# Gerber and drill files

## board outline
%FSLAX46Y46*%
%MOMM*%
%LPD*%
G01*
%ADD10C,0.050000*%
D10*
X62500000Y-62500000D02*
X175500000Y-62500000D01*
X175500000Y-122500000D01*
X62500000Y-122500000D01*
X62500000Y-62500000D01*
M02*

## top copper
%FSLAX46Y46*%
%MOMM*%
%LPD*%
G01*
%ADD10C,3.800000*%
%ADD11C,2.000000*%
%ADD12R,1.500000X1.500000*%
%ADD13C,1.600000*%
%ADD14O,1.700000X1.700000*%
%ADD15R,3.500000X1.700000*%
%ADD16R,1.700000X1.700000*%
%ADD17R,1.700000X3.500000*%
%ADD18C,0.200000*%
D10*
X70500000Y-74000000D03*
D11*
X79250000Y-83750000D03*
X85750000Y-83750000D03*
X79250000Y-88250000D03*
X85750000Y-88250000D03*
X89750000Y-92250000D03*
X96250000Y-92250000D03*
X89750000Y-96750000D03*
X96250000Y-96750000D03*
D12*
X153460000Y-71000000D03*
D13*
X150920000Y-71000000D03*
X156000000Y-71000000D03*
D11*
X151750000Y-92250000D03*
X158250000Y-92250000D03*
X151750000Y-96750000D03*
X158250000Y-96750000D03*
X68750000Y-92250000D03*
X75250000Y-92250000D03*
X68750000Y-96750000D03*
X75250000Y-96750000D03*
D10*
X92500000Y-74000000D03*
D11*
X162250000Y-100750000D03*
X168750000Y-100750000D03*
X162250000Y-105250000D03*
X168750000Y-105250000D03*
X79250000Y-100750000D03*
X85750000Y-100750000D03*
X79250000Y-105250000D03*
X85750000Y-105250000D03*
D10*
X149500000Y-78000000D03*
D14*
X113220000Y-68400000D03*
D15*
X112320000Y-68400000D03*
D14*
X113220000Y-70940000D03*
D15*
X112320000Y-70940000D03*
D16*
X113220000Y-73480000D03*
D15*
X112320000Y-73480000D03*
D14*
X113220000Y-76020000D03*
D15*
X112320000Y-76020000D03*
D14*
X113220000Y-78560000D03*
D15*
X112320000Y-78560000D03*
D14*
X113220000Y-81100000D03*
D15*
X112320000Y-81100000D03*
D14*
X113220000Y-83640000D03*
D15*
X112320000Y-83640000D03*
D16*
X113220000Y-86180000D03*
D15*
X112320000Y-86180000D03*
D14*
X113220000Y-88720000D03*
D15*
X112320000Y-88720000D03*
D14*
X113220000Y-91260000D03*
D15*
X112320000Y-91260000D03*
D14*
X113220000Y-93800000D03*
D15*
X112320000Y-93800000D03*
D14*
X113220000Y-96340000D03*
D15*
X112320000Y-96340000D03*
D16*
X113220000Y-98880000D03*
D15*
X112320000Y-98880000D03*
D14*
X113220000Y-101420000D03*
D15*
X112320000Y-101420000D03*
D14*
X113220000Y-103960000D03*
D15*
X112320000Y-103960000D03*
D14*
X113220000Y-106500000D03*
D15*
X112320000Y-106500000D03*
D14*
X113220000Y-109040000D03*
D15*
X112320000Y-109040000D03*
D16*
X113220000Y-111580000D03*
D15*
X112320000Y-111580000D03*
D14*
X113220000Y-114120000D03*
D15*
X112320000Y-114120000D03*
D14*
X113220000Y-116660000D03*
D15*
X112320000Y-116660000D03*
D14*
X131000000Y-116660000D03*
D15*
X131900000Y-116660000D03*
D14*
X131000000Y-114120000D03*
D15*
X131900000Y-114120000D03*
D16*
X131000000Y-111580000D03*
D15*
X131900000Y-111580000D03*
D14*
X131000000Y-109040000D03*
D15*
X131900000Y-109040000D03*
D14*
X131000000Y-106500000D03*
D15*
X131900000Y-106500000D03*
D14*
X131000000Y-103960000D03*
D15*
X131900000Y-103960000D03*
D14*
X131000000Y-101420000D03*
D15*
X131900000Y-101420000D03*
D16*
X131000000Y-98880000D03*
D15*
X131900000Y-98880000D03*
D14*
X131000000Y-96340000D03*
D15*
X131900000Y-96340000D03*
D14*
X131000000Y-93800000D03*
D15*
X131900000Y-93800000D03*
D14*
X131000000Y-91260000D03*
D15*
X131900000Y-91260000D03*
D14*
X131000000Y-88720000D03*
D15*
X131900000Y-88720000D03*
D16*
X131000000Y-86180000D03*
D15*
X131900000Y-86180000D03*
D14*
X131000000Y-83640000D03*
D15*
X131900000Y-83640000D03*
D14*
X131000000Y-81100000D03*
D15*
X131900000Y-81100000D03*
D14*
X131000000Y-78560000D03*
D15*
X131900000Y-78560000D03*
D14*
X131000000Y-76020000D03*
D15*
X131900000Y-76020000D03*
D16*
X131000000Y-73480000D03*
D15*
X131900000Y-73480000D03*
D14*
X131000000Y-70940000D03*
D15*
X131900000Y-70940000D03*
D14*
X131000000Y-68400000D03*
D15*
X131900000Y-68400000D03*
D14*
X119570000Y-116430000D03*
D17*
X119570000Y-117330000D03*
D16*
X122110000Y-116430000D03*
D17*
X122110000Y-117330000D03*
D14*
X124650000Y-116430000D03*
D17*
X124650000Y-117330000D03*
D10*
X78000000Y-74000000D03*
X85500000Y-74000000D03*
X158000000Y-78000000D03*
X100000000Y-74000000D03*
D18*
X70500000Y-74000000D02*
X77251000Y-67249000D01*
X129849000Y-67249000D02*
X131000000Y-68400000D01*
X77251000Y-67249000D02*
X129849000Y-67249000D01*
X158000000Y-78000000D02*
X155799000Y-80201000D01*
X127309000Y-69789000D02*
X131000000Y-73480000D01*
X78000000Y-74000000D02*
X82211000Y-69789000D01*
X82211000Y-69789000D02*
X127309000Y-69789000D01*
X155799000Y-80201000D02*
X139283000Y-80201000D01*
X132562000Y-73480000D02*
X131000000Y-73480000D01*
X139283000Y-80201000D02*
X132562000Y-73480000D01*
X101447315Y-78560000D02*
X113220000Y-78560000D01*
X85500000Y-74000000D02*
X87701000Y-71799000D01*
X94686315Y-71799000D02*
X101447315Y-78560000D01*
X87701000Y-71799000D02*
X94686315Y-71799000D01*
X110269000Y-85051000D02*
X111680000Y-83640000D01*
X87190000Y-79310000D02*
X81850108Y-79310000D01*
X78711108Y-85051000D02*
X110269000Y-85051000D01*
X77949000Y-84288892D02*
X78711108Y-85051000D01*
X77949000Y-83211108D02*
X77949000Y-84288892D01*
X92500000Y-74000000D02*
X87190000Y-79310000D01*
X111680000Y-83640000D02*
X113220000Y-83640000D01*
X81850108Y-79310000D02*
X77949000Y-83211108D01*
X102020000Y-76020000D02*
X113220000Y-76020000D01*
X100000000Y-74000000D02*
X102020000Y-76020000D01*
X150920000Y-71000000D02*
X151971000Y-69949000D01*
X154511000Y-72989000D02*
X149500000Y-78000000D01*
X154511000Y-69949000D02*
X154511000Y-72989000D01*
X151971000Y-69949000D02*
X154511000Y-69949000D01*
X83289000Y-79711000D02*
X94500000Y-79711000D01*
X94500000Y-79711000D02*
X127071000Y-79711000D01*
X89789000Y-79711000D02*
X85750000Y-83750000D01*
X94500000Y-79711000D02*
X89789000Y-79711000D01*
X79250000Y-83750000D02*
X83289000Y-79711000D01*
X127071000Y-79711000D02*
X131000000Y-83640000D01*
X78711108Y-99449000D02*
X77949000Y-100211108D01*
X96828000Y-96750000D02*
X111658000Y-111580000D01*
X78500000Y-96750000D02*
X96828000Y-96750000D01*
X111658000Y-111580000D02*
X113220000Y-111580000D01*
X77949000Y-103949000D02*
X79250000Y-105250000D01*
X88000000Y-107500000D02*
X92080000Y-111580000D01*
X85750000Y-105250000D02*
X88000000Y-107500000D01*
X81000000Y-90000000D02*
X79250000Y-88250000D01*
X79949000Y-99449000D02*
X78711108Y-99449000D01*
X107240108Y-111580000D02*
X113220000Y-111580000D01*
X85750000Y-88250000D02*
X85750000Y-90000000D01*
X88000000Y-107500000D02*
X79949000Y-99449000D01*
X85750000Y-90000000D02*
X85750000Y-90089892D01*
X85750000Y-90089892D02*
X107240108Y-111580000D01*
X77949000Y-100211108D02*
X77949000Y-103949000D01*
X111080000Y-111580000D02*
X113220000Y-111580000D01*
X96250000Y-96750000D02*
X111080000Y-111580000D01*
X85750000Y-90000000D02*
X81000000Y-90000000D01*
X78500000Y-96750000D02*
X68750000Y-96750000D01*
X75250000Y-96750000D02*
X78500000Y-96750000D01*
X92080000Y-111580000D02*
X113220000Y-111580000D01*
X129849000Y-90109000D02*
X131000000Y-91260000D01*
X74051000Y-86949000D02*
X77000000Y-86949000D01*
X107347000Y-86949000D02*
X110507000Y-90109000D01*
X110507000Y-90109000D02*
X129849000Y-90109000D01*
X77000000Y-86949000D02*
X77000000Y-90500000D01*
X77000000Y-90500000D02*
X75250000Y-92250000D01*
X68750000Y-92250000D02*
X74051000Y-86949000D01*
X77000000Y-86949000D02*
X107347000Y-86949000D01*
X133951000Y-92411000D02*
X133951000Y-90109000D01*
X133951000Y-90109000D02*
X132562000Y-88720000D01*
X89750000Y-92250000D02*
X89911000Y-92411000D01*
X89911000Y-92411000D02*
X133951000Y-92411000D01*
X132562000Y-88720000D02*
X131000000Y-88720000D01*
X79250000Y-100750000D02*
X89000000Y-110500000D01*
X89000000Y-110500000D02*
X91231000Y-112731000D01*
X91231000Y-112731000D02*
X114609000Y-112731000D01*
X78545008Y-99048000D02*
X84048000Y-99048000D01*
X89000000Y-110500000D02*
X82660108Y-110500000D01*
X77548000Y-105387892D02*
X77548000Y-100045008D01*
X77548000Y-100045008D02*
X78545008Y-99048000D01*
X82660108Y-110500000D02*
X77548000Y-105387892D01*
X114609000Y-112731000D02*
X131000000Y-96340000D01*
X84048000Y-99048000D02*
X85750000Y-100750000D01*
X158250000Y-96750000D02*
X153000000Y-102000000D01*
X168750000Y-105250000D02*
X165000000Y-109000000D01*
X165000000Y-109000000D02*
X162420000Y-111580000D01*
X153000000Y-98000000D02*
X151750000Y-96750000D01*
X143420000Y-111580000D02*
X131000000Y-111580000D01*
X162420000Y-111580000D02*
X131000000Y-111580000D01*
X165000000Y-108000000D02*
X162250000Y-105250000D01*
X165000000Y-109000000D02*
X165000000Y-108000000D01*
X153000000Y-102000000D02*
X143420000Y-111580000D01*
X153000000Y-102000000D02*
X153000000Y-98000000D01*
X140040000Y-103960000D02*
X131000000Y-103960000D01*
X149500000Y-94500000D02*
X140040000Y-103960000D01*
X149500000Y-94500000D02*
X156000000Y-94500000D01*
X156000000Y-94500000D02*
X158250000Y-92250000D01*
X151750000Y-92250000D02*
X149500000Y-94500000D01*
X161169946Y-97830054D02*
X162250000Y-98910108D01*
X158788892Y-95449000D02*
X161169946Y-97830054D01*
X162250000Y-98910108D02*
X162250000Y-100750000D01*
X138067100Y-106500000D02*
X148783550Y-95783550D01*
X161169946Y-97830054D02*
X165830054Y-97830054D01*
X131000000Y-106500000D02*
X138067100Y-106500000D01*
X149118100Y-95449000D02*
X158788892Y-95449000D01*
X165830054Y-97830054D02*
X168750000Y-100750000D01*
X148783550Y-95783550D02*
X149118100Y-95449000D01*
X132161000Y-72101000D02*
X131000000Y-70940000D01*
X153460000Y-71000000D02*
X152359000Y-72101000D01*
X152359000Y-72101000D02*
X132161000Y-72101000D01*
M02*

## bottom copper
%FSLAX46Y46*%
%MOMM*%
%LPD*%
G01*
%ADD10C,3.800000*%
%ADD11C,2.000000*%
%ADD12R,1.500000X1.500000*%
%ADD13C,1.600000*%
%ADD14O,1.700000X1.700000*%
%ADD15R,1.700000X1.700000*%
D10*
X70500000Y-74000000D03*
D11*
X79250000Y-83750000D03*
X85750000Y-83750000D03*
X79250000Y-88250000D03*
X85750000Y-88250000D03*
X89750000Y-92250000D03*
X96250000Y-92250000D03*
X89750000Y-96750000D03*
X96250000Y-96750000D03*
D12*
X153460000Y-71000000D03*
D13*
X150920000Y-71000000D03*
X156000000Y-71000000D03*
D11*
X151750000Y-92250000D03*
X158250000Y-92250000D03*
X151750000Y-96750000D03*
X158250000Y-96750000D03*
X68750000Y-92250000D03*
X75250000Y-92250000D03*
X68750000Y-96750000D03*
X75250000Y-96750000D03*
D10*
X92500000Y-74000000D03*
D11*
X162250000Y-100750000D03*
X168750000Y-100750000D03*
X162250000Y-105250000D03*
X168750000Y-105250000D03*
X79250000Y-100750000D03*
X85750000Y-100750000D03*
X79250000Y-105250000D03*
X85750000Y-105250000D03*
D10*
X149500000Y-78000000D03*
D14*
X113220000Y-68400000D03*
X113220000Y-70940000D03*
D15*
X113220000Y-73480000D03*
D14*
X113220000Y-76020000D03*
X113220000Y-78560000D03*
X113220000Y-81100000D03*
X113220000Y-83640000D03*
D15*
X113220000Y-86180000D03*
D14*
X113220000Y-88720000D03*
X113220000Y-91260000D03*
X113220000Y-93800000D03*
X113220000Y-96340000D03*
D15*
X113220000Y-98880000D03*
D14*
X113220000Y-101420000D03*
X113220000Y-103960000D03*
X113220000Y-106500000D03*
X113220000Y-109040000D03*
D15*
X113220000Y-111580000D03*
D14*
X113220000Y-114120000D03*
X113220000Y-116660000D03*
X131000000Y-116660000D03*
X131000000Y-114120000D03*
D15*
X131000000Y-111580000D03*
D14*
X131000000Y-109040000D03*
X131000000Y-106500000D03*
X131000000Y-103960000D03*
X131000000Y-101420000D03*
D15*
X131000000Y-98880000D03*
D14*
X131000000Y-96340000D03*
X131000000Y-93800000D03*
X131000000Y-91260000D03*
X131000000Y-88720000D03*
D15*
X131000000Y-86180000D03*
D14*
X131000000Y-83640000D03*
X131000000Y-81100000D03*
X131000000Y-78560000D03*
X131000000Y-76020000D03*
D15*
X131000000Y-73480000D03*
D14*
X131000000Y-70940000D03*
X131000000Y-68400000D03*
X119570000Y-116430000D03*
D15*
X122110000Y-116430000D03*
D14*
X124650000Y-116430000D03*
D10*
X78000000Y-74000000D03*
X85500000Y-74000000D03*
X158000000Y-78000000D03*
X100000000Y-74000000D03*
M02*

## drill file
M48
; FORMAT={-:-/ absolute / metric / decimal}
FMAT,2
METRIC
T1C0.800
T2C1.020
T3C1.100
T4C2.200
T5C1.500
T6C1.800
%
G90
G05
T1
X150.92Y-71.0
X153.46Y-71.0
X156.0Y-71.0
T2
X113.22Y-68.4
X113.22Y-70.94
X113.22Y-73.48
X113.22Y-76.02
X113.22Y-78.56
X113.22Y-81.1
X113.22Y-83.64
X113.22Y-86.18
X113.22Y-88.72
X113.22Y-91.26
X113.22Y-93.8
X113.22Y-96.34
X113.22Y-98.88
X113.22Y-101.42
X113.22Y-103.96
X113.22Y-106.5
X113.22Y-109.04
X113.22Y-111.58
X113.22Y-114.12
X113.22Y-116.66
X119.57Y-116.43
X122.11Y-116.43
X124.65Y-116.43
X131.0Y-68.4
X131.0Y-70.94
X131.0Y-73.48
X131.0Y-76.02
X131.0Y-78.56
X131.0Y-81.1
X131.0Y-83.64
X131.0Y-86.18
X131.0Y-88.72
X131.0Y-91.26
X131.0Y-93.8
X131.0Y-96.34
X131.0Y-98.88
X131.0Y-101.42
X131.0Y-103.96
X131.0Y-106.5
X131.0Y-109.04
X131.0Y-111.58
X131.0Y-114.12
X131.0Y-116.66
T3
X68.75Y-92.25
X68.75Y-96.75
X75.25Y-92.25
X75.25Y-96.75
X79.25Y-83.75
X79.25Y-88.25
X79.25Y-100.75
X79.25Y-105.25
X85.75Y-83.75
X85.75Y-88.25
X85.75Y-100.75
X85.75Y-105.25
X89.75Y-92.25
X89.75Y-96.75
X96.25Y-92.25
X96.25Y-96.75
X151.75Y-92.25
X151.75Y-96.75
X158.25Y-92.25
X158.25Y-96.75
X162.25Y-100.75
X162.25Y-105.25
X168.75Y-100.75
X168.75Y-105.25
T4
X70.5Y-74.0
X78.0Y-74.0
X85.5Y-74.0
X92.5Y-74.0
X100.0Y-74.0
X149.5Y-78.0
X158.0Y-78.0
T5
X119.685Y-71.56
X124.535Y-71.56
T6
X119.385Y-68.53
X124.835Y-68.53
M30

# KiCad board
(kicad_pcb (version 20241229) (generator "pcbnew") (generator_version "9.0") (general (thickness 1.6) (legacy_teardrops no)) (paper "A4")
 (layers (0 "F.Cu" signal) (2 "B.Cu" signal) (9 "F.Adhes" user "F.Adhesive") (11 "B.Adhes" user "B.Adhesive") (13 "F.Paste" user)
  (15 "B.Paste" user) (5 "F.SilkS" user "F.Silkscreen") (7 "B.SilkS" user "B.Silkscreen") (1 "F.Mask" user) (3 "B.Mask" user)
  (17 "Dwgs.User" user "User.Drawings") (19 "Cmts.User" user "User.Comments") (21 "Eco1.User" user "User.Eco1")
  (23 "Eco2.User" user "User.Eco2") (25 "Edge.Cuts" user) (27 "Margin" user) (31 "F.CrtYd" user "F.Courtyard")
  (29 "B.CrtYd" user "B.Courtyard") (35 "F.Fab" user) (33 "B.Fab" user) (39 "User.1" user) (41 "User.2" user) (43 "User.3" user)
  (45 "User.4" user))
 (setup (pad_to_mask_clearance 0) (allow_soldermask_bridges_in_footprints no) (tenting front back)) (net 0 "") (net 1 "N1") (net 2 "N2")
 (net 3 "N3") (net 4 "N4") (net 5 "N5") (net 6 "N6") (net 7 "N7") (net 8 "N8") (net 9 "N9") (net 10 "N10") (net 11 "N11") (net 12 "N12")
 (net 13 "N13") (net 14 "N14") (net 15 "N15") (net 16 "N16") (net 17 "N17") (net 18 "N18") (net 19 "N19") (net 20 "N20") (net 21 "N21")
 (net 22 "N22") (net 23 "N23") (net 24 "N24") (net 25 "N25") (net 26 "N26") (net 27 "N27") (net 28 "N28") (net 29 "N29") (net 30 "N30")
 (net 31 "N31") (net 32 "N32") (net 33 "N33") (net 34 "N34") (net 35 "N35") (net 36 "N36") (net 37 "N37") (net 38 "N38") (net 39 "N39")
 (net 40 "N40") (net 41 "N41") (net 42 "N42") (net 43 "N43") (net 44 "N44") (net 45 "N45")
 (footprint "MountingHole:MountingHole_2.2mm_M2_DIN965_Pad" (layer "F.Cu") (at 70.5 74)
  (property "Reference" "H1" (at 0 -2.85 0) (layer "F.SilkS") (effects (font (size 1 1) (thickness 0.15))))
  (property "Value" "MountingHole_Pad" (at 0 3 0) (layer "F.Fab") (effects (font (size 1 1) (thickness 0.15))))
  (pad "1" thru_hole circle (at 0 0) (size 3.8 3.8) (drill 2.2) (layers "*.Cu" "*.Mask") (remove_unused_layers no) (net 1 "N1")
   (zone_connect 2)))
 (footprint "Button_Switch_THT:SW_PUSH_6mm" (layer "F.Cu") (at 79.25 83.75)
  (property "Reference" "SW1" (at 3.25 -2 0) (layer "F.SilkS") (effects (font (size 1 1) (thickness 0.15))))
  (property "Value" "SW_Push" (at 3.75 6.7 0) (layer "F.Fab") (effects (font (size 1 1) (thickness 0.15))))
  (pad "1" thru_hole circle (at 0 0 90) (size 2 2) (drill 1.1) (layers "*.Cu" "*.Mask") (remove_unused_layers no) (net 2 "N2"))
  (pad "1" thru_hole circle (at 6.5 0 90) (size 2 2) (drill 1.1) (layers "*.Cu" "*.Mask") (remove_unused_layers no) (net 2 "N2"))
  (pad "2" thru_hole circle (at 0 4.5 90) (size 2 2) (drill 1.1) (layers "*.Cu" "*.Mask") (remove_unused_layers no) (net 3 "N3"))
  (pad "2" thru_hole circle (at 6.5 4.5 90) (size 2 2) (drill 1.1) (layers "*.Cu" "*.Mask") (remove_unused_layers no) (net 3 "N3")))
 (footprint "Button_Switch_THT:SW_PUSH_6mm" (layer "F.Cu") (at 89.75 92.25)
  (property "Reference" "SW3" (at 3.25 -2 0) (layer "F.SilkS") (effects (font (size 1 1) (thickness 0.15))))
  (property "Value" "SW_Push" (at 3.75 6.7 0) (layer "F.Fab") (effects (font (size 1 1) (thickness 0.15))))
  (pad "1" thru_hole circle (at 0 0 90) (size 2 2) (drill 1.1) (layers "*.Cu" "*.Mask") (remove_unused_layers no) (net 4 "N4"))
  (pad "1" thru_hole circle (at 6.5 0 90) (size 2 2) (drill 1.1) (layers "*.Cu" "*.Mask") (remove_unused_layers no) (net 4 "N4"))
  (pad "2" thru_hole circle (at 0 4.5 90) (size 2 2) (drill 1.1) (layers "*.Cu" "*.Mask") (remove_unused_layers no) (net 3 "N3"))
  (pad "2" thru_hole circle (at 6.5 4.5 90) (size 2 2) (drill 1.1) (layers "*.Cu" "*.Mask") (remove_unused_layers no) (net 3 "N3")))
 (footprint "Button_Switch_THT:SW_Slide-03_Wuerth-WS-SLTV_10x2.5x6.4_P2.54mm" (layer "F.Cu") (at 153.46 71)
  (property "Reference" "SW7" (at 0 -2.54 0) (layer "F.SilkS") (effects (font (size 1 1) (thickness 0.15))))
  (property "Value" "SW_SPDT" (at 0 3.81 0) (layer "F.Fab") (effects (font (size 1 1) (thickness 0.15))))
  (pad "1" thru_hole rect (at 0 0) (size 1.5 1.5) (drill 0.8) (layers "*.Cu" "*.Mask") (remove_unused_layers no) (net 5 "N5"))
  (pad "2" thru_hole circle (at -2.54 0) (size 1.6 1.6) (drill 0.8) (layers "*.Cu" "*.Mask") (remove_unused_layers no) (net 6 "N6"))
  (pad "3" thru_hole circle (at 2.54 0) (size 1.6 1.6) (drill 0.8) (layers "*.Cu" "*.Mask") (remove_unused_layers no) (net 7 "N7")))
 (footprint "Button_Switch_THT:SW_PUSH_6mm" (layer "F.Cu") (at 151.75 92.25)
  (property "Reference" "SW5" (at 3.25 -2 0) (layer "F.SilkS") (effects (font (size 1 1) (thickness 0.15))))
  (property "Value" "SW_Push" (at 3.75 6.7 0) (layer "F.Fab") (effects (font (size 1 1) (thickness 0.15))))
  (pad "1" thru_hole circle (at 0 0 90) (size 2 2) (drill 1.1) (layers "*.Cu" "*.Mask") (remove_unused_layers no) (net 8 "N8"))
  (pad "1" thru_hole circle (at 6.5 0 90) (size 2 2) (drill 1.1) (layers "*.Cu" "*.Mask") (remove_unused_layers no) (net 8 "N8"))
  (pad "2" thru_hole circle (at 0 4.5 90) (size 2 2) (drill 1.1) (layers "*.Cu" "*.Mask") (remove_unused_layers no) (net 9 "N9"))
  (pad "2" thru_hole circle (at 6.5 4.5 90) (size 2 2) (drill 1.1) (layers "*.Cu" "*.Mask") (remove_unused_layers no) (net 9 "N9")))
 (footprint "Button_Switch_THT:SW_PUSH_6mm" (layer "F.Cu") (at 68.75 92.25)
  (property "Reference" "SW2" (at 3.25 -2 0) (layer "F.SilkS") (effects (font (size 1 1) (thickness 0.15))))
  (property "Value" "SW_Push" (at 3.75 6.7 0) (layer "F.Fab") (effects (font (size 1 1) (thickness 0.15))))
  (pad "1" thru_hole circle (at 0 0 90) (size 2 2) (drill 1.1) (layers "*.Cu" "*.Mask") (remove_unused_layers no) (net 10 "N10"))
  (pad "1" thru_hole circle (at 6.5 0 90) (size 2 2) (drill 1.1) (layers "*.Cu" "*.Mask") (remove_unused_layers no) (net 10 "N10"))
  (pad "2" thru_hole circle (at 0 4.5 90) (size 2 2) (drill 1.1) (layers "*.Cu" "*.Mask") (remove_unused_layers no) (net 3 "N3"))
  (pad "2" thru_hole circle (at 6.5 4.5 90) (size 2 2) (drill 1.1) (layers "*.Cu" "*.Mask") (remove_unused_layers no) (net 3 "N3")))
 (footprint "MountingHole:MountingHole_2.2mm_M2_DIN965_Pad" (layer "F.Cu") (at 92.5 74)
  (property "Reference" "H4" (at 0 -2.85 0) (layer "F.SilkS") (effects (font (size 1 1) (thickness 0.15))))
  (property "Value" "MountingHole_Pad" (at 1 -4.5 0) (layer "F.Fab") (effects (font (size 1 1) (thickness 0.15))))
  (pad "1" thru_hole circle (at 0 0) (size 3.8 3.8) (drill 2.2) (layers "*.Cu" "*.Mask") (remove_unused_layers no) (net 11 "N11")
   (zone_connect 2)))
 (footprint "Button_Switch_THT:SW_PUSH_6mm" (layer "F.Cu") (at 162.25 100.75)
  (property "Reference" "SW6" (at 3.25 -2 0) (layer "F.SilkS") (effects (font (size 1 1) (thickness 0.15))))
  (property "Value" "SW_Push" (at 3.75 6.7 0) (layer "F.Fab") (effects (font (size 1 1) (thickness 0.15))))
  (pad "1" thru_hole circle (at 0 0 90) (size 2 2) (drill 1.1) (layers "*.Cu" "*.Mask") (remove_unused_layers no) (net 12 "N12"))
  (pad "1" thru_hole circle (at 6.5 0 90) (size 2 2) (drill 1.1) (layers "*.Cu" "*.Mask") (remove_unused_layers no) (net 12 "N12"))
  (pad "2" thru_hole circle (at 0 4.5 90) (size 2 2) (drill 1.1) (layers "*.Cu" "*.Mask") (remove_unused_layers no) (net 9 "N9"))
  (pad "2" thru_hole circle (at 6.5 4.5 90) (size 2 2) (drill 1.1) (layers "*.Cu" "*.Mask") (remove_unused_layers no) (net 9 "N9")))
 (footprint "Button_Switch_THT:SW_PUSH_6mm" (layer "F.Cu") (at 79.25 100.75)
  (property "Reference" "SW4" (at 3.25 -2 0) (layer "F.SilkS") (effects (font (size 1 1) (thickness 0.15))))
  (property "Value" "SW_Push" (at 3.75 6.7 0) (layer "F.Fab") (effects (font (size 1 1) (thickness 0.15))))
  (pad "1" thru_hole circle (at 0 0 90) (size 2 2) (drill 1.1) (layers "*.Cu" "*.Mask") (remove_unused_layers no) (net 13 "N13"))
  (pad "1" thru_hole circle (at 6.5 0 90) (size 2 2) (drill 1.1) (layers "*.Cu" "*.Mask") (remove_unused_layers no) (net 13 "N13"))
  (pad "2" thru_hole circle (at 0 4.5 90) (size 2 2) (drill 1.1) (layers "*.Cu" "*.Mask") (remove_unused_layers no) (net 3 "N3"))
  (pad "2" thru_hole circle (at 6.5 4.5 90) (size 2 2) (drill 1.1) (layers "*.Cu" "*.Mask") (remove_unused_layers no) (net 3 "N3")))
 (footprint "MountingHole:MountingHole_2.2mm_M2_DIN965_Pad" (layer "F.Cu") (at 149.5 78)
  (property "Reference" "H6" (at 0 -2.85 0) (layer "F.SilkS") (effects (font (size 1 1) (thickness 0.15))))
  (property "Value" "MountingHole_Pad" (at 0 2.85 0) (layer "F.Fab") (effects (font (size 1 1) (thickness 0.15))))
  (pad "1" thru_hole circle (at 0 0) (size 3.8 3.8) (drill 2.2) (layers "*.Cu" "*.Mask") (remove_unused_layers no) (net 6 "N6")
   (zone_connect 2)))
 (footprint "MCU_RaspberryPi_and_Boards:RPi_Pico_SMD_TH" (layer "F.Cu") (at 122.11 92.53)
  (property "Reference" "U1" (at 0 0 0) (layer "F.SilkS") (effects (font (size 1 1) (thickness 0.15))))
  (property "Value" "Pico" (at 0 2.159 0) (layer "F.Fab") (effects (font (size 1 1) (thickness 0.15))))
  (pad "" np_thru_hole oval (at -2.725 -24) (size 1.8 1.8) (drill 1.8) (layers "*.Cu" "*.Mask"))
  (pad "" np_thru_hole oval (at -2.425 -20.97) (size 1.5 1.5) (drill 1.5) (layers "*.Cu" "*.Mask"))
  (pad "" np_thru_hole oval (at 2.425 -20.97) (size 1.5 1.5) (drill 1.5) (layers "*.Cu" "*.Mask"))
  (pad "" np_thru_hole oval (at 2.725 -24) (size 1.8 1.8) (drill 1.8) (layers "*.Cu" "*.Mask"))
  (pad "1" thru_hole oval (at -8.89 -24.13) (size 1.7 1.7) (drill 1.02) (layers "*.Cu" "*.Mask") (remove_unused_layers no) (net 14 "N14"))
  (pad "1" smd rect (at -8.89 -24.13) (size 3.5 1.7) (drill (offset -0.9 0)) (layers "F.Cu" "F.Mask") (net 14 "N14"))
  (pad "2" thru_hole oval (at -8.89 -21.59) (size 1.7 1.7) (drill 1.02) (layers "*.Cu" "*.Mask") (remove_unused_layers no) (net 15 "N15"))
  (pad "2" smd rect (at -8.89 -21.59) (size 3.5 1.7) (drill (offset -0.9 0)) (layers "F.Cu" "F.Mask") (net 15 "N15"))
  (pad "3" thru_hole rect (at -8.89 -19.05) (size 1.7 1.7) (drill 1.02) (layers "*.Cu" "*.Mask") (remove_unused_layers no) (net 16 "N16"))
  (pad "3" smd rect (at -8.89 -19.05) (size 3.5 1.7) (drill (offset -0.9 0)) (layers "F.Cu" "F.Mask") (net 16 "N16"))
  (pad "4" thru_hole oval (at -8.89 -16.51) (size 1.7 1.7) (drill 1.02) (layers "*.Cu" "*.Mask") (remove_unused_layers no) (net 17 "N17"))
  (pad "4" smd rect (at -8.89 -16.51) (size 3.5 1.7) (drill (offset -0.9 0)) (layers "F.Cu" "F.Mask") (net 17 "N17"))
  (pad "5" thru_hole oval (at -8.89 -13.97) (size 1.7 1.7) (drill 1.02) (layers "*.Cu" "*.Mask") (remove_unused_layers no) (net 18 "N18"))
  (pad "5" smd rect (at -8.89 -13.97) (size 3.5 1.7) (drill (offset -0.9 0)) (layers "F.Cu" "F.Mask") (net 18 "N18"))
  (pad "6" thru_hole oval (at -8.89 -11.43) (size 1.7 1.7) (drill 1.02) (layers "*.Cu" "*.Mask") (remove_unused_layers no) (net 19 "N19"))
  (pad "6" smd rect (at -8.89 -11.43) (size 3.5 1.7) (drill (offset -0.9 0)) (layers "F.Cu" "F.Mask") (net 19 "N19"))
  (pad "7" thru_hole oval (at -8.89 -8.89) (size 1.7 1.7) (drill 1.02) (layers "*.Cu" "*.Mask") (remove_unused_layers no) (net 11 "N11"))
  (pad "7" smd rect (at -8.89 -8.89) (size 3.5 1.7) (drill (offset -0.9 0)) (layers "F.Cu" "F.Mask") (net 11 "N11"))
  (pad "8" thru_hole rect (at -8.89 -6.35) (size 1.7 1.7) (drill 1.02) (layers "*.Cu" "*.Mask") (remove_unused_layers no) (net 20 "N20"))
  (pad "8" smd rect (at -8.89 -6.35) (size 3.5 1.7) (drill (offset -0.9 0)) (layers "F.Cu" "F.Mask") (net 20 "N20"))
  (pad "9" thru_hole oval (at -8.89 -3.81) (size 1.7 1.7) (drill 1.02) (layers "*.Cu" "*.Mask") (remove_unused_layers no) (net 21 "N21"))
  (pad "9" smd rect (at -8.89 -3.81) (size 3.5 1.7) (drill (offset -0.9 0)) (layers "F.Cu" "F.Mask") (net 21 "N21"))
  (pad "10" thru_hole oval (at -8.89 -1.27) (size 1.7 1.7) (drill 1.02) (layers "*.Cu" "*.Mask") (remove_unused_layers no) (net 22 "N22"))
  (pad "10" smd rect (at -8.89 -1.27) (size 3.5 1.7) (drill (offset -0.9 0)) (layers "F.Cu" "F.Mask") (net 22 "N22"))
  (pad "11" thru_hole oval (at -8.89 1.27) (size 1.7 1.7) (drill 1.02) (layers "*.Cu" "*.Mask") (remove_unused_layers no) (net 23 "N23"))
  (pad "11" smd rect (at -8.89 1.27) (size 3.5 1.7) (drill (offset -0.9 0)) (layers "F.Cu" "F.Mask") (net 23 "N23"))
  (pad "12" thru_hole oval (at -8.89 3.81) (size 1.7 1.7) (drill 1.02) (layers "*.Cu" "*.Mask") (remove_unused_layers no) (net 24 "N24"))
  (pad "12" smd rect (at -8.89 3.81) (size 3.5 1.7) (drill (offset -0.9 0)) (layers "F.Cu" "F.Mask") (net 24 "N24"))
  (pad "13" thru_hole rect (at -8.89 6.35) (size 1.7 1.7) (drill 1.02) (layers "*.Cu" "*.Mask") (remove_unused_layers no) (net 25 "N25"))
  (pad "13" smd rect (at -8.89 6.35) (size 3.5 1.7) (drill (offset -0.9 0)) (layers "F.Cu" "F.Mask") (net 25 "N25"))
  (pad "14" thru_hole oval (at -8.89 8.89) (size 1.7 1.7) (drill 1.02) (layers "*.Cu" "*.Mask") (remove_unused_layers no) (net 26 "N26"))
  (pad "14" smd rect (at -8.89 8.89) (size 3.5 1.7) (drill (offset -0.9 0)) (layers "F.Cu" "F.Mask") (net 26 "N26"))
  (pad "15" thru_hole oval (at -8.89 11.43) (size 1.7 1.7) (drill 1.02) (layers "*.Cu" "*.Mask") (remove_unused_layers no) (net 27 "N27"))
  (pad "15" smd rect (at -8.89 11.43) (size 3.5 1.7) (drill (offset -0.9 0)) (layers "F.Cu" "F.Mask") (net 27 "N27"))
  (pad "16" thru_hole oval (at -8.89 13.97) (size 1.7 1.7) (drill 1.02) (layers "*.Cu" "*.Mask") (remove_unused_layers no) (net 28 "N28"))
  (pad "16" smd rect (at -8.89 13.97) (size 3.5 1.7) (drill (offset -0.9 0)) (layers "F.Cu" "F.Mask") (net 28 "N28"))
  (pad "17" thru_hole oval (at -8.89 16.51) (size 1.7 1.7) (drill 1.02) (layers "*.Cu" "*.Mask") (remove_unused_layers no) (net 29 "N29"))
  (pad "17" smd rect (at -8.89 16.51) (size 3.5 1.7) (drill (offset -0.9 0)) (layers "F.Cu" "F.Mask") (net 29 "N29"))
  (pad "18" thru_hole rect (at -8.89 19.05) (size 1.7 1.7) (drill 1.02) (layers "*.Cu" "*.Mask") (remove_unused_layers no) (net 3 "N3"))
  (pad "18" smd rect (at -8.89 19.05) (size 3.5 1.7) (drill (offset -0.9 0)) (layers "F.Cu" "F.Mask") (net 3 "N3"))
  (pad "19" thru_hole oval (at -8.89 21.59) (size 1.7 1.7) (drill 1.02) (layers "*.Cu" "*.Mask") (remove_unused_layers no) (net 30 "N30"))
  (pad "19" smd rect (at -8.89 21.59) (size 3.5 1.7) (drill (offset -0.9 0)) (layers "F.Cu" "F.Mask") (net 30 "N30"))
  (pad "20" thru_hole oval (at -8.89 24.13) (size 1.7 1.7) (drill 1.02) (layers "*.Cu" "*.Mask") (remove_unused_layers no) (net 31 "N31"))
  (pad "20" smd rect (at -8.89 24.13) (size 3.5 1.7) (drill (offset -0.9 0)) (layers "F.Cu" "F.Mask") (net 31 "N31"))
  (pad "21" thru_hole oval (at 8.89 24.13) (size 1.7 1.7) (drill 1.02) (layers "*.Cu" "*.Mask") (remove_unused_layers no) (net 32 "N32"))
  (pad "21" smd rect (at 8.89 24.13) (size 3.5 1.7) (drill (offset 0.9 0)) (layers "F.Cu" "F.Mask") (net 32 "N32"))
  (pad "22" thru_hole oval (at 8.89 21.59) (size 1.7 1.7) (drill 1.02) (layers "*.Cu" "*.Mask") (remove_unused_layers no) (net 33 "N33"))
  (pad "22" smd rect (at 8.89 21.59) (size 3.5 1.7) (drill (offset 0.9 0)) (layers "F.Cu" "F.Mask") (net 33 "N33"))
  (pad "23" thru_hole rect (at 8.89 19.05) (size 1.7 1.7) (drill 1.02) (layers "*.Cu" "*.Mask") (remove_unused_layers no) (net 9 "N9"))
  (pad "23" smd rect (at 8.89 19.05) (size 3.5 1.7) (drill (offset 0.9 0)) (layers "F.Cu" "F.Mask") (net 9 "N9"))
  (pad "24" thru_hole oval (at 8.89 16.51) (size 1.7 1.7) (drill 1.02) (layers "*.Cu" "*.Mask") (remove_unused_layers no) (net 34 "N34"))
  (pad "24" smd rect (at 8.89 16.51) (size 3.5 1.7) (drill (offset 0.9 0)) (layers "F.Cu" "F.Mask") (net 34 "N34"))
  (pad "25" thru_hole oval (at 8.89 13.97) (size 1.7 1.7) (drill 1.02) (layers "*.Cu" "*.Mask") (remove_unused_layers no) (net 12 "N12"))
  (pad "25" smd rect (at 8.89 13.97) (size 3.5 1.7) (drill (offset 0.9 0)) (layers "F.Cu" "F.Mask") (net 12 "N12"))
  (pad "26" thru_hole oval (at 8.89 11.43) (size 1.7 1.7) (drill 1.02) (layers "*.Cu" "*.Mask") (remove_unused_layers no) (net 8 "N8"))
  (pad "26" smd rect (at 8.89 11.43) (size 3.5 1.7) (drill (offset 0.9 0)) (layers "F.Cu" "F.Mask") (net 8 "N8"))
  (pad "27" thru_hole oval (at 8.89 8.89) (size 1.7 1.7) (drill 1.02) (layers "*.Cu" "*.Mask") (remove_unused_layers no) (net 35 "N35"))
  (pad "27" smd rect (at 8.89 8.89) (size 3.5 1.7) (drill (offset 0.9 0)) (layers "F.Cu" "F.Mask") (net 35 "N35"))
  (pad "28" thru_hole rect (at 8.89 6.35) (size 1.7 1.7) (drill 1.02) (layers "*.Cu" "*.Mask") (remove_unused_layers no) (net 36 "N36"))
  (pad "28" smd rect (at 8.89 6.35) (size 3.5 1.7) (drill (offset 0.9 0)) (layers "F.Cu" "F.Mask") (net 36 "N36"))
  (pad "29" thru_hole oval (at 8.89 3.81) (size 1.7 1.7) (drill 1.02) (layers "*.Cu" "*.Mask") (remove_unused_layers no) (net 13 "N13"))
  (pad "29" smd rect (at 8.89 3.81) (size 3.5 1.7) (drill (offset 0.9 0)) (layers "F.Cu" "F.Mask") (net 13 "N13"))
  (pad "30" thru_hole oval (at 8.89 1.27) (size 1.7 1.7) (drill 1.02) (layers "*.Cu" "*.Mask") (remove_unused_layers no) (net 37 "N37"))
  (pad "30" smd rect (at 8.89 1.27) (size 3.5 1.7) (drill (offset 0.9 0)) (layers "F.Cu" "F.Mask") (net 37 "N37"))
  (pad "31" thru_hole oval (at 8.89 -1.27) (size 1.7 1.7) (drill 1.02) (layers "*.Cu" "*.Mask") (remove_unused_layers no) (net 10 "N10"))
  (pad "31" smd rect (at 8.89 -1.27) (size 3.5 1.7) (drill (offset 0.9 0)) (layers "F.Cu" "F.Mask") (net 10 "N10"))
  (pad "32" thru_hole oval (at 8.89 -3.81) (size 1.7 1.7) (drill 1.02) (layers "*.Cu" "*.Mask") (remove_unused_layers no) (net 4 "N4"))
  (pad "32" smd rect (at 8.89 -3.81) (size 3.5 1.7) (drill (offset 0.9 0)) (layers "F.Cu" "F.Mask") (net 4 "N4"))
  (pad "33" thru_hole rect (at 8.89 -6.35) (size 1.7 1.7) (drill 1.02) (layers "*.Cu" "*.Mask") (remove_unused_layers no) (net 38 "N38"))
  (pad "33" smd rect (at 8.89 -6.35) (size 3.5 1.7) (drill (offset 0.9 0)) (layers "F.Cu" "F.Mask") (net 38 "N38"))
  (pad "34" thru_hole oval (at 8.89 -8.89) (size 1.7 1.7) (drill 1.02) (layers "*.Cu" "*.Mask") (remove_unused_layers no) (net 2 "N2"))
  (pad "34" smd rect (at 8.89 -8.89) (size 3.5 1.7) (drill (offset 0.9 0)) (layers "F.Cu" "F.Mask") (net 2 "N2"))
  (pad "35" thru_hole oval (at 8.89 -11.43) (size 1.7 1.7) (drill 1.02) (layers "*.Cu" "*.Mask") (remove_unused_layers no) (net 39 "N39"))
  (pad "35" smd rect (at 8.89 -11.43) (size 3.5 1.7) (drill (offset 0.9 0)) (layers "F.Cu" "F.Mask") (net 39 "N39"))
  (pad "36" thru_hole oval (at 8.89 -13.97) (size 1.7 1.7) (drill 1.02) (layers "*.Cu" "*.Mask") (remove_unused_layers no) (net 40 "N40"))
  (pad "36" smd rect (at 8.89 -13.97) (size 3.5 1.7) (drill (offset 0.9 0)) (layers "F.Cu" "F.Mask") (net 40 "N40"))
  (pad "37" thru_hole oval (at 8.89 -16.51) (size 1.7 1.7) (drill 1.02) (layers "*.Cu" "*.Mask") (remove_unused_layers no) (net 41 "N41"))
  (pad "37" smd rect (at 8.89 -16.51) (size 3.5 1.7) (drill (offset 0.9 0)) (layers "F.Cu" "F.Mask") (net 41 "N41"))
  (pad "38" thru_hole rect (at 8.89 -19.05) (size 1.7 1.7) (drill 1.02) (layers "*.Cu" "*.Mask") (remove_unused_layers no) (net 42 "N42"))
  (pad "38" smd rect (at 8.89 -19.05) (size 3.5 1.7) (drill (offset 0.9 0)) (layers "F.Cu" "F.Mask") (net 42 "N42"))
  (pad "39" thru_hole oval (at 8.89 -21.59) (size 1.7 1.7) (drill 1.02) (layers "*.Cu" "*.Mask") (remove_unused_layers no) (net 5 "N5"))
  (pad "39" smd rect (at 8.89 -21.59) (size 3.5 1.7) (drill (offset 0.9 0)) (layers "F.Cu" "F.Mask") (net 5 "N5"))
  (pad "40" thru_hole oval (at 8.89 -24.13) (size 1.7 1.7) (drill 1.02) (layers "*.Cu" "*.Mask") (remove_unused_layers no) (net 1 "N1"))
  (pad "40" smd rect (at 8.89 -24.13) (size 3.5 1.7) (drill (offset 0.9 0)) (layers "F.Cu" "F.Mask") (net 1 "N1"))
  (pad "41" thru_hole oval (at -2.54 23.9) (size 1.7 1.7) (drill 1.02) (layers "*.Cu" "*.Mask") (remove_unused_layers no) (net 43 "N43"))
  (pad "41" smd rect (at -2.54 23.9 90) (size 3.5 1.7) (drill (offset -0.9 0)) (layers "F.Cu" "F.Mask") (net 43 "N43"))
  (pad "42" thru_hole rect (at 0 23.9) (size 1.7 1.7) (drill 1.02) (layers "*.Cu" "*.Mask") (remove_unused_layers no) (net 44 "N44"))
  (pad "42" smd rect (at 0 23.9 90) (size 3.5 1.7) (drill (offset -0.9 0)) (layers "F.Cu" "F.Mask") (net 44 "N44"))
  (pad "43" thru_hole oval (at 2.54 23.9) (size 1.7 1.7) (drill 1.02) (layers "*.Cu" "*.Mask") (remove_unused_layers no) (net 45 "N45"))
  (pad "43" smd rect (at 2.54 23.9 90) (size 3.5 1.7) (drill (offset -0.9 0)) (layers "F.Cu" "F.Mask") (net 45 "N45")))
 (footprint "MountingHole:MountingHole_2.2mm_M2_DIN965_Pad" (layer "F.Cu") (at 78 74)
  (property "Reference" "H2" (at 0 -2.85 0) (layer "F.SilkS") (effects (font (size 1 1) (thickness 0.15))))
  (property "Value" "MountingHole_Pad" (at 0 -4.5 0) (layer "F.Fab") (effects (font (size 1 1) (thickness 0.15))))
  (pad "1" thru_hole circle (at 0 0) (size 3.8 3.8) (drill 2.2) (layers "*.Cu" "*.Mask") (remove_unused_layers no) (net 42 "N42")
   (zone_connect 2)))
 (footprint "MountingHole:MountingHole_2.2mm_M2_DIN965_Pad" (layer "F.Cu") (at 85.5 74)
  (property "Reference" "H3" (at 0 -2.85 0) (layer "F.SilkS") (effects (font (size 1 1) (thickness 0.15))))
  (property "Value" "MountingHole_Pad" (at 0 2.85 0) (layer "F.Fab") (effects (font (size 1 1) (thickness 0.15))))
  (pad "1" thru_hole circle (at 0 0) (size 3.8 3.8) (drill 2.2) (layers "*.Cu" "*.Mask") (remove_unused_layers no) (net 18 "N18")
   (zone_connect 2)))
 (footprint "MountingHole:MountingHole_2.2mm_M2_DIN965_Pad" (layer "F.Cu") (at 158 78)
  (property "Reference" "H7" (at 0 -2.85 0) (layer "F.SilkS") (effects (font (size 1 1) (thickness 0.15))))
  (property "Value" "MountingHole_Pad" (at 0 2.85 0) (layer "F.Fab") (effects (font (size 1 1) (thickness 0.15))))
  (pad "1" thru_hole circle (at 0 0) (size 3.8 3.8) (drill 2.2) (layers "*.Cu" "*.Mask") (remove_unused_layers no) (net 42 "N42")
   (zone_connect 2)))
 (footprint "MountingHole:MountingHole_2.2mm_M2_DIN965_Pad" (layer "F.Cu") (at 100 74)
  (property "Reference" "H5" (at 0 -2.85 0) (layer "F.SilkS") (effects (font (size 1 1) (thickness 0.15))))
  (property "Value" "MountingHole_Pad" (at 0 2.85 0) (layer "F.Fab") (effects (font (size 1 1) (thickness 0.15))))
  (pad "1" thru_hole circle (at 0 0) (size 3.8 3.8) (drill 2.2) (layers "*.Cu" "*.Mask") (remove_unused_layers no) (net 17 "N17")
   (zone_connect 2)))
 (gr_rect (start 62.5 62.5) (end 175.5 122.5) (stroke (width 0.05) (type default)) (fill no) (layer "Edge.Cuts"))
 (segment (start 70.5 74) (end 77.251 67.249) (width 0.2) (layer "F.Cu") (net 1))
 (segment (start 129.849 67.249) (end 131 68.4) (width 0.2) (layer "F.Cu") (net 1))
 (segment (start 77.251 67.249) (end 129.849 67.249) (width 0.2) (layer "F.Cu") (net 1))
 (segment (start 158 78) (end 155.799 80.201) (width 0.2) (layer "F.Cu") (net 42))
 (segment (start 127.309 69.789) (end 131 73.48) (width 0.2) (layer "F.Cu") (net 42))
 (segment (start 78 74) (end 82.211 69.789) (width 0.2) (layer "F.Cu") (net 42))
 (segment (start 82.211 69.789) (end 127.309 69.789) (width 0.2) (layer "F.Cu") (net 42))
 (segment (start 155.799 80.201) (end 139.283 80.201) (width 0.2) (layer "F.Cu") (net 42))
 (segment (start 132.562 73.48) (end 131 73.48) (width 0.2) (layer "F.Cu") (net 42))
 (segment (start 139.283 80.201) (end 132.562 73.48) (width 0.2) (layer "F.Cu") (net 42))
 (segment (start 101.447315 78.56) (end 113.22 78.56) (width 0.2) (layer "F.Cu") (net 18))
 (segment (start 85.5 74) (end 87.701 71.799) (width 0.2) (layer "F.Cu") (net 18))
 (segment (start 94.686315 71.799) (end 101.447315 78.56) (width 0.2) (layer "F.Cu") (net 18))
 (segment (start 87.701 71.799) (end 94.686315 71.799) (width 0.2) (layer "F.Cu") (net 18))
 (segment (start 110.269 85.051) (end 111.68 83.64) (width 0.2) (layer "F.Cu") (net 11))
 (segment (start 87.19 79.31) (end 81.850108 79.31) (width 0.2) (layer "F.Cu") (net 11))
 (segment (start 78.711108 85.051) (end 110.269 85.051) (width 0.2) (layer "F.Cu") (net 11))
 (segment (start 77.949 84.288892) (end 78.711108 85.051) (width 0.2) (layer "F.Cu") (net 11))
 (segment (start 77.949 83.211108) (end 77.949 84.288892) (width 0.2) (layer "F.Cu") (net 11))
 (segment (start 92.5 74) (end 87.19 79.31) (width 0.2) (layer "F.Cu") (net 11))
 (segment (start 111.68 83.64) (end 113.22 83.64) (width 0.2) (layer "F.Cu") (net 11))
 (segment (start 81.850108 79.31) (end 77.949 83.211108) (width 0.2) (layer "F.Cu") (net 11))
 (segment (start 102.02 76.02) (end 113.22 76.02) (width 0.2) (layer "F.Cu") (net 17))
 (segment (start 100 74) (end 102.02 76.02) (width 0.2) (layer "F.Cu") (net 17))
 (segment (start 150.92 71) (end 151.971 69.949) (width 0.2) (layer "F.Cu") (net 6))
 (segment (start 154.511 72.989) (end 149.5 78) (width 0.2) (layer "F.Cu") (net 6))
 (segment (start 154.511 69.949) (end 154.511 72.989) (width 0.2) (layer "F.Cu") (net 6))
 (segment (start 151.971 69.949) (end 154.511 69.949) (width 0.2) (layer "F.Cu") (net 6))
 (segment (start 83.289 79.711) (end 94.5 79.711) (width 0.2) (layer "F.Cu") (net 2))
 (segment (start 94.5 79.711) (end 127.071 79.711) (width 0.2) (layer "F.Cu") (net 2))
 (segment (start 89.789 79.711) (end 85.75 83.75) (width 0.2) (layer "F.Cu") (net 2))
 (segment (start 94.5 79.711) (end 89.789 79.711) (width 0.2) (layer "F.Cu") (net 2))
 (segment (start 79.25 83.75) (end 83.289 79.711) (width 0.2) (layer "F.Cu") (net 2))
 (segment (start 127.071 79.711) (end 131 83.64) (width 0.2) (layer "F.Cu") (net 2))
 (segment (start 78.711108 99.449) (end 77.949 100.211108) (width 0.2) (layer "F.Cu") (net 3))
 (segment (start 96.828 96.75) (end 111.658 111.58) (width 0.2) (layer "F.Cu") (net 3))
 (segment (start 78.5 96.75) (end 96.828 96.75) (width 0.2) (layer "F.Cu") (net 3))
 (segment (start 111.658 111.58) (end 113.22 111.58) (width 0.2) (layer "F.Cu") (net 3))
 (segment (start 77.949 103.949) (end 79.25 105.25) (width 0.2) (layer "F.Cu") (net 3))
 (segment (start 88 107.5) (end 92.08 111.58) (width 0.2) (layer "F.Cu") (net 3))
 (segment (start 85.75 105.25) (end 88 107.5) (width 0.2) (layer "F.Cu") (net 3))
 (segment (start 81 90) (end 79.25 88.25) (width 0.2) (layer "F.Cu") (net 3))
 (segment (start 79.949 99.449) (end 78.711108 99.449) (width 0.2) (layer "F.Cu") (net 3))
 (segment (start 107.240108 111.58) (end 113.22 111.58) (width 0.2) (layer "F.Cu") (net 3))
 (segment (start 85.75 88.25) (end 85.75 90) (width 0.2) (layer "F.Cu") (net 3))
 (segment (start 88 107.5) (end 79.949 99.449) (width 0.2) (layer "F.Cu") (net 3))
 (segment (start 85.75 90) (end 85.75 90.089892) (width 0.2) (layer "F.Cu") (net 3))
 (segment (start 85.75 90.089892) (end 107.240108 111.58) (width 0.2) (layer "F.Cu") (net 3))
 (segment (start 77.949 100.211108) (end 77.949 103.949) (width 0.2) (layer "F.Cu") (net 3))
 (segment (start 111.08 111.58) (end 113.22 111.58) (width 0.2) (layer "F.Cu") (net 3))
 (segment (start 96.25 96.75) (end 111.08 111.58) (width 0.2) (layer "F.Cu") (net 3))
 (segment (start 85.75 90) (end 81 90) (width 0.2) (layer "F.Cu") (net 3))
 (segment (start 78.5 96.75) (end 68.75 96.75) (width 0.2) (layer "F.Cu") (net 3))
 (segment (start 75.25 96.75) (end 78.5 96.75) (width 0.2) (layer "F.Cu") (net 3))
 (segment (start 92.08 111.58) (end 113.22 111.58) (width 0.2) (layer "F.Cu") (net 3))
 (segment (start 129.849 90.109) (end 131 91.26) (width 0.2) (layer "F.Cu") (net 10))
 (segment (start 74.051 86.949) (end 77 86.949) (width 0.2) (layer "F.Cu") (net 10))
 (segment (start 107.347 86.949) (end 110.507 90.109) (width 0.2) (layer "F.Cu") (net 10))
 (segment (start 110.507 90.109) (end 129.849 90.109) (width 0.2) (layer "F.Cu") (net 10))
 (segment (start 77 86.949) (end 77 90.5) (width 0.2) (layer "F.Cu") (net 10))
 (segment (start 77 90.5) (end 75.25 92.25) (width 0.2) (layer "F.Cu") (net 10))
 (segment (start 68.75 92.25) (end 74.051 86.949) (width 0.2) (layer "F.Cu") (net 10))
 (segment (start 77 86.949) (end 107.347 86.949) (width 0.2) (layer "F.Cu") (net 10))
 (segment (start 133.951 92.411) (end 133.951 90.109) (width 0.2) (layer "F.Cu") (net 4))
 (segment (start 133.951 90.109) (end 132.562 88.72) (width 0.2) (layer "F.Cu") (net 4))
 (segment (start 89.75 92.25) (end 89.911 92.411) (width 0.2) (layer "F.Cu") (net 4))
 (segment (start 89.911 92.411) (end 133.951 92.411) (width 0.2) (layer "F.Cu") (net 4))
 (segment (start 132.562 88.72) (end 131 88.72) (width 0.2) (layer "F.Cu") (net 4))
 (segment (start 79.25 100.75) (end 89 110.5) (width 0.2) (layer "F.Cu") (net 13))
 (segment (start 89 110.5) (end 91.231 112.731) (width 0.2) (layer "F.Cu") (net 13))
 (segment (start 91.231 112.731) (end 114.609 112.731) (width 0.2) (layer "F.Cu") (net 13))
 (segment (start 78.545008 99.048) (end 84.048 99.048) (width 0.2) (layer "F.Cu") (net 13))
 (segment (start 89 110.5) (end 82.660108 110.5) (width 0.2) (layer "F.Cu") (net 13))
 (segment (start 77.548 105.387892) (end 77.548 100.045008) (width 0.2) (layer "F.Cu") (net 13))
 (segment (start 77.548 100.045008) (end 78.545008 99.048) (width 0.2) (layer "F.Cu") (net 13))
 (segment (start 82.660108 110.5) (end 77.548 105.387892) (width 0.2) (layer "F.Cu") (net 13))
 (segment (start 114.609 112.731) (end 131 96.34) (width 0.2) (layer "F.Cu") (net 13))
 (segment (start 84.048 99.048) (end 85.75 100.75) (width 0.2) (layer "F.Cu") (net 13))
 (segment (start 158.25 96.75) (end 153 102) (width 0.2) (layer "F.Cu") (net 9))
 (segment (start 168.75 105.25) (end 165 109) (width 0.2) (layer "F.Cu") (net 9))
 (segment (start 165 109) (end 162.42 111.58) (width 0.2) (layer "F.Cu") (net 9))
 (segment (start 153 98) (end 151.75 96.75) (width 0.2) (layer "F.Cu") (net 9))
 (segment (start 143.42 111.58) (end 131 111.58) (width 0.2) (layer "F.Cu") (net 9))
 (segment (start 162.42 111.58) (end 131 111.58) (width 0.2) (layer "F.Cu") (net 9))
 (segment (start 165 108) (end 162.25 105.25) (width 0.2) (layer "F.Cu") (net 9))
 (segment (start 165 109) (end 165 108) (width 0.2) (layer "F.Cu") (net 9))
 (segment (start 153 102) (end 143.42 111.58) (width 0.2) (layer "F.Cu") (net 9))
 (segment (start 153 102) (end 153 98) (width 0.2) (layer "F.Cu") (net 9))
 (segment (start 140.04 103.96) (end 131 103.96) (width 0.2) (layer "F.Cu") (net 8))
 (segment (start 149.5 94.5) (end 140.04 103.96) (width 0.2) (layer "F.Cu") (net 8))
 (segment (start 149.5 94.5) (end 156 94.5) (width 0.2) (layer "F.Cu") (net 8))
 (segment (start 156 94.5) (end 158.25 92.25) (width 0.2) (layer "F.Cu") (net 8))
 (segment (start 151.75 92.25) (end 149.5 94.5) (width 0.2) (layer "F.Cu") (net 8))
 (segment (start 161.169946 97.830054) (end 162.25 98.910108) (width 0.2) (layer "F.Cu") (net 12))
 (segment (start 158.788892 95.449) (end 161.169946 97.830054) (width 0.2) (layer "F.Cu") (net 12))
 (segment (start 162.25 98.910108) (end 162.25 100.75) (width 0.2) (layer "F.Cu") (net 12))
 (segment (start 138.0671 106.5) (end 148.78355 95.78355) (width 0.2) (layer "F.Cu") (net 12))
 (segment (start 161.169946 97.830054) (end 165.830054 97.830054) (width 0.2) (layer "F.Cu") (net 12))
 (segment (start 131 106.5) (end 138.0671 106.5) (width 0.2) (layer "F.Cu") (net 12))
 (segment (start 149.1181 95.449) (end 158.788892 95.449) (width 0.2) (layer "F.Cu") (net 12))
 (segment (start 165.830054 97.830054) (end 168.75 100.75) (width 0.2) (layer "F.Cu") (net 12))
 (segment (start 148.78355 95.78355) (end 149.1181 95.449) (width 0.2) (layer "F.Cu") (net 12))
 (segment (start 132.161 72.101) (end 131 70.94) (width 0.2) (layer "F.Cu") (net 5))
 (segment (start 153.46 71) (end 152.359 72.101) (width 0.2) (layer "F.Cu") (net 5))
 (segment (start 152.359 72.101) (end 132.161 72.101) (width 0.2) (layer "F.Cu") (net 5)))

